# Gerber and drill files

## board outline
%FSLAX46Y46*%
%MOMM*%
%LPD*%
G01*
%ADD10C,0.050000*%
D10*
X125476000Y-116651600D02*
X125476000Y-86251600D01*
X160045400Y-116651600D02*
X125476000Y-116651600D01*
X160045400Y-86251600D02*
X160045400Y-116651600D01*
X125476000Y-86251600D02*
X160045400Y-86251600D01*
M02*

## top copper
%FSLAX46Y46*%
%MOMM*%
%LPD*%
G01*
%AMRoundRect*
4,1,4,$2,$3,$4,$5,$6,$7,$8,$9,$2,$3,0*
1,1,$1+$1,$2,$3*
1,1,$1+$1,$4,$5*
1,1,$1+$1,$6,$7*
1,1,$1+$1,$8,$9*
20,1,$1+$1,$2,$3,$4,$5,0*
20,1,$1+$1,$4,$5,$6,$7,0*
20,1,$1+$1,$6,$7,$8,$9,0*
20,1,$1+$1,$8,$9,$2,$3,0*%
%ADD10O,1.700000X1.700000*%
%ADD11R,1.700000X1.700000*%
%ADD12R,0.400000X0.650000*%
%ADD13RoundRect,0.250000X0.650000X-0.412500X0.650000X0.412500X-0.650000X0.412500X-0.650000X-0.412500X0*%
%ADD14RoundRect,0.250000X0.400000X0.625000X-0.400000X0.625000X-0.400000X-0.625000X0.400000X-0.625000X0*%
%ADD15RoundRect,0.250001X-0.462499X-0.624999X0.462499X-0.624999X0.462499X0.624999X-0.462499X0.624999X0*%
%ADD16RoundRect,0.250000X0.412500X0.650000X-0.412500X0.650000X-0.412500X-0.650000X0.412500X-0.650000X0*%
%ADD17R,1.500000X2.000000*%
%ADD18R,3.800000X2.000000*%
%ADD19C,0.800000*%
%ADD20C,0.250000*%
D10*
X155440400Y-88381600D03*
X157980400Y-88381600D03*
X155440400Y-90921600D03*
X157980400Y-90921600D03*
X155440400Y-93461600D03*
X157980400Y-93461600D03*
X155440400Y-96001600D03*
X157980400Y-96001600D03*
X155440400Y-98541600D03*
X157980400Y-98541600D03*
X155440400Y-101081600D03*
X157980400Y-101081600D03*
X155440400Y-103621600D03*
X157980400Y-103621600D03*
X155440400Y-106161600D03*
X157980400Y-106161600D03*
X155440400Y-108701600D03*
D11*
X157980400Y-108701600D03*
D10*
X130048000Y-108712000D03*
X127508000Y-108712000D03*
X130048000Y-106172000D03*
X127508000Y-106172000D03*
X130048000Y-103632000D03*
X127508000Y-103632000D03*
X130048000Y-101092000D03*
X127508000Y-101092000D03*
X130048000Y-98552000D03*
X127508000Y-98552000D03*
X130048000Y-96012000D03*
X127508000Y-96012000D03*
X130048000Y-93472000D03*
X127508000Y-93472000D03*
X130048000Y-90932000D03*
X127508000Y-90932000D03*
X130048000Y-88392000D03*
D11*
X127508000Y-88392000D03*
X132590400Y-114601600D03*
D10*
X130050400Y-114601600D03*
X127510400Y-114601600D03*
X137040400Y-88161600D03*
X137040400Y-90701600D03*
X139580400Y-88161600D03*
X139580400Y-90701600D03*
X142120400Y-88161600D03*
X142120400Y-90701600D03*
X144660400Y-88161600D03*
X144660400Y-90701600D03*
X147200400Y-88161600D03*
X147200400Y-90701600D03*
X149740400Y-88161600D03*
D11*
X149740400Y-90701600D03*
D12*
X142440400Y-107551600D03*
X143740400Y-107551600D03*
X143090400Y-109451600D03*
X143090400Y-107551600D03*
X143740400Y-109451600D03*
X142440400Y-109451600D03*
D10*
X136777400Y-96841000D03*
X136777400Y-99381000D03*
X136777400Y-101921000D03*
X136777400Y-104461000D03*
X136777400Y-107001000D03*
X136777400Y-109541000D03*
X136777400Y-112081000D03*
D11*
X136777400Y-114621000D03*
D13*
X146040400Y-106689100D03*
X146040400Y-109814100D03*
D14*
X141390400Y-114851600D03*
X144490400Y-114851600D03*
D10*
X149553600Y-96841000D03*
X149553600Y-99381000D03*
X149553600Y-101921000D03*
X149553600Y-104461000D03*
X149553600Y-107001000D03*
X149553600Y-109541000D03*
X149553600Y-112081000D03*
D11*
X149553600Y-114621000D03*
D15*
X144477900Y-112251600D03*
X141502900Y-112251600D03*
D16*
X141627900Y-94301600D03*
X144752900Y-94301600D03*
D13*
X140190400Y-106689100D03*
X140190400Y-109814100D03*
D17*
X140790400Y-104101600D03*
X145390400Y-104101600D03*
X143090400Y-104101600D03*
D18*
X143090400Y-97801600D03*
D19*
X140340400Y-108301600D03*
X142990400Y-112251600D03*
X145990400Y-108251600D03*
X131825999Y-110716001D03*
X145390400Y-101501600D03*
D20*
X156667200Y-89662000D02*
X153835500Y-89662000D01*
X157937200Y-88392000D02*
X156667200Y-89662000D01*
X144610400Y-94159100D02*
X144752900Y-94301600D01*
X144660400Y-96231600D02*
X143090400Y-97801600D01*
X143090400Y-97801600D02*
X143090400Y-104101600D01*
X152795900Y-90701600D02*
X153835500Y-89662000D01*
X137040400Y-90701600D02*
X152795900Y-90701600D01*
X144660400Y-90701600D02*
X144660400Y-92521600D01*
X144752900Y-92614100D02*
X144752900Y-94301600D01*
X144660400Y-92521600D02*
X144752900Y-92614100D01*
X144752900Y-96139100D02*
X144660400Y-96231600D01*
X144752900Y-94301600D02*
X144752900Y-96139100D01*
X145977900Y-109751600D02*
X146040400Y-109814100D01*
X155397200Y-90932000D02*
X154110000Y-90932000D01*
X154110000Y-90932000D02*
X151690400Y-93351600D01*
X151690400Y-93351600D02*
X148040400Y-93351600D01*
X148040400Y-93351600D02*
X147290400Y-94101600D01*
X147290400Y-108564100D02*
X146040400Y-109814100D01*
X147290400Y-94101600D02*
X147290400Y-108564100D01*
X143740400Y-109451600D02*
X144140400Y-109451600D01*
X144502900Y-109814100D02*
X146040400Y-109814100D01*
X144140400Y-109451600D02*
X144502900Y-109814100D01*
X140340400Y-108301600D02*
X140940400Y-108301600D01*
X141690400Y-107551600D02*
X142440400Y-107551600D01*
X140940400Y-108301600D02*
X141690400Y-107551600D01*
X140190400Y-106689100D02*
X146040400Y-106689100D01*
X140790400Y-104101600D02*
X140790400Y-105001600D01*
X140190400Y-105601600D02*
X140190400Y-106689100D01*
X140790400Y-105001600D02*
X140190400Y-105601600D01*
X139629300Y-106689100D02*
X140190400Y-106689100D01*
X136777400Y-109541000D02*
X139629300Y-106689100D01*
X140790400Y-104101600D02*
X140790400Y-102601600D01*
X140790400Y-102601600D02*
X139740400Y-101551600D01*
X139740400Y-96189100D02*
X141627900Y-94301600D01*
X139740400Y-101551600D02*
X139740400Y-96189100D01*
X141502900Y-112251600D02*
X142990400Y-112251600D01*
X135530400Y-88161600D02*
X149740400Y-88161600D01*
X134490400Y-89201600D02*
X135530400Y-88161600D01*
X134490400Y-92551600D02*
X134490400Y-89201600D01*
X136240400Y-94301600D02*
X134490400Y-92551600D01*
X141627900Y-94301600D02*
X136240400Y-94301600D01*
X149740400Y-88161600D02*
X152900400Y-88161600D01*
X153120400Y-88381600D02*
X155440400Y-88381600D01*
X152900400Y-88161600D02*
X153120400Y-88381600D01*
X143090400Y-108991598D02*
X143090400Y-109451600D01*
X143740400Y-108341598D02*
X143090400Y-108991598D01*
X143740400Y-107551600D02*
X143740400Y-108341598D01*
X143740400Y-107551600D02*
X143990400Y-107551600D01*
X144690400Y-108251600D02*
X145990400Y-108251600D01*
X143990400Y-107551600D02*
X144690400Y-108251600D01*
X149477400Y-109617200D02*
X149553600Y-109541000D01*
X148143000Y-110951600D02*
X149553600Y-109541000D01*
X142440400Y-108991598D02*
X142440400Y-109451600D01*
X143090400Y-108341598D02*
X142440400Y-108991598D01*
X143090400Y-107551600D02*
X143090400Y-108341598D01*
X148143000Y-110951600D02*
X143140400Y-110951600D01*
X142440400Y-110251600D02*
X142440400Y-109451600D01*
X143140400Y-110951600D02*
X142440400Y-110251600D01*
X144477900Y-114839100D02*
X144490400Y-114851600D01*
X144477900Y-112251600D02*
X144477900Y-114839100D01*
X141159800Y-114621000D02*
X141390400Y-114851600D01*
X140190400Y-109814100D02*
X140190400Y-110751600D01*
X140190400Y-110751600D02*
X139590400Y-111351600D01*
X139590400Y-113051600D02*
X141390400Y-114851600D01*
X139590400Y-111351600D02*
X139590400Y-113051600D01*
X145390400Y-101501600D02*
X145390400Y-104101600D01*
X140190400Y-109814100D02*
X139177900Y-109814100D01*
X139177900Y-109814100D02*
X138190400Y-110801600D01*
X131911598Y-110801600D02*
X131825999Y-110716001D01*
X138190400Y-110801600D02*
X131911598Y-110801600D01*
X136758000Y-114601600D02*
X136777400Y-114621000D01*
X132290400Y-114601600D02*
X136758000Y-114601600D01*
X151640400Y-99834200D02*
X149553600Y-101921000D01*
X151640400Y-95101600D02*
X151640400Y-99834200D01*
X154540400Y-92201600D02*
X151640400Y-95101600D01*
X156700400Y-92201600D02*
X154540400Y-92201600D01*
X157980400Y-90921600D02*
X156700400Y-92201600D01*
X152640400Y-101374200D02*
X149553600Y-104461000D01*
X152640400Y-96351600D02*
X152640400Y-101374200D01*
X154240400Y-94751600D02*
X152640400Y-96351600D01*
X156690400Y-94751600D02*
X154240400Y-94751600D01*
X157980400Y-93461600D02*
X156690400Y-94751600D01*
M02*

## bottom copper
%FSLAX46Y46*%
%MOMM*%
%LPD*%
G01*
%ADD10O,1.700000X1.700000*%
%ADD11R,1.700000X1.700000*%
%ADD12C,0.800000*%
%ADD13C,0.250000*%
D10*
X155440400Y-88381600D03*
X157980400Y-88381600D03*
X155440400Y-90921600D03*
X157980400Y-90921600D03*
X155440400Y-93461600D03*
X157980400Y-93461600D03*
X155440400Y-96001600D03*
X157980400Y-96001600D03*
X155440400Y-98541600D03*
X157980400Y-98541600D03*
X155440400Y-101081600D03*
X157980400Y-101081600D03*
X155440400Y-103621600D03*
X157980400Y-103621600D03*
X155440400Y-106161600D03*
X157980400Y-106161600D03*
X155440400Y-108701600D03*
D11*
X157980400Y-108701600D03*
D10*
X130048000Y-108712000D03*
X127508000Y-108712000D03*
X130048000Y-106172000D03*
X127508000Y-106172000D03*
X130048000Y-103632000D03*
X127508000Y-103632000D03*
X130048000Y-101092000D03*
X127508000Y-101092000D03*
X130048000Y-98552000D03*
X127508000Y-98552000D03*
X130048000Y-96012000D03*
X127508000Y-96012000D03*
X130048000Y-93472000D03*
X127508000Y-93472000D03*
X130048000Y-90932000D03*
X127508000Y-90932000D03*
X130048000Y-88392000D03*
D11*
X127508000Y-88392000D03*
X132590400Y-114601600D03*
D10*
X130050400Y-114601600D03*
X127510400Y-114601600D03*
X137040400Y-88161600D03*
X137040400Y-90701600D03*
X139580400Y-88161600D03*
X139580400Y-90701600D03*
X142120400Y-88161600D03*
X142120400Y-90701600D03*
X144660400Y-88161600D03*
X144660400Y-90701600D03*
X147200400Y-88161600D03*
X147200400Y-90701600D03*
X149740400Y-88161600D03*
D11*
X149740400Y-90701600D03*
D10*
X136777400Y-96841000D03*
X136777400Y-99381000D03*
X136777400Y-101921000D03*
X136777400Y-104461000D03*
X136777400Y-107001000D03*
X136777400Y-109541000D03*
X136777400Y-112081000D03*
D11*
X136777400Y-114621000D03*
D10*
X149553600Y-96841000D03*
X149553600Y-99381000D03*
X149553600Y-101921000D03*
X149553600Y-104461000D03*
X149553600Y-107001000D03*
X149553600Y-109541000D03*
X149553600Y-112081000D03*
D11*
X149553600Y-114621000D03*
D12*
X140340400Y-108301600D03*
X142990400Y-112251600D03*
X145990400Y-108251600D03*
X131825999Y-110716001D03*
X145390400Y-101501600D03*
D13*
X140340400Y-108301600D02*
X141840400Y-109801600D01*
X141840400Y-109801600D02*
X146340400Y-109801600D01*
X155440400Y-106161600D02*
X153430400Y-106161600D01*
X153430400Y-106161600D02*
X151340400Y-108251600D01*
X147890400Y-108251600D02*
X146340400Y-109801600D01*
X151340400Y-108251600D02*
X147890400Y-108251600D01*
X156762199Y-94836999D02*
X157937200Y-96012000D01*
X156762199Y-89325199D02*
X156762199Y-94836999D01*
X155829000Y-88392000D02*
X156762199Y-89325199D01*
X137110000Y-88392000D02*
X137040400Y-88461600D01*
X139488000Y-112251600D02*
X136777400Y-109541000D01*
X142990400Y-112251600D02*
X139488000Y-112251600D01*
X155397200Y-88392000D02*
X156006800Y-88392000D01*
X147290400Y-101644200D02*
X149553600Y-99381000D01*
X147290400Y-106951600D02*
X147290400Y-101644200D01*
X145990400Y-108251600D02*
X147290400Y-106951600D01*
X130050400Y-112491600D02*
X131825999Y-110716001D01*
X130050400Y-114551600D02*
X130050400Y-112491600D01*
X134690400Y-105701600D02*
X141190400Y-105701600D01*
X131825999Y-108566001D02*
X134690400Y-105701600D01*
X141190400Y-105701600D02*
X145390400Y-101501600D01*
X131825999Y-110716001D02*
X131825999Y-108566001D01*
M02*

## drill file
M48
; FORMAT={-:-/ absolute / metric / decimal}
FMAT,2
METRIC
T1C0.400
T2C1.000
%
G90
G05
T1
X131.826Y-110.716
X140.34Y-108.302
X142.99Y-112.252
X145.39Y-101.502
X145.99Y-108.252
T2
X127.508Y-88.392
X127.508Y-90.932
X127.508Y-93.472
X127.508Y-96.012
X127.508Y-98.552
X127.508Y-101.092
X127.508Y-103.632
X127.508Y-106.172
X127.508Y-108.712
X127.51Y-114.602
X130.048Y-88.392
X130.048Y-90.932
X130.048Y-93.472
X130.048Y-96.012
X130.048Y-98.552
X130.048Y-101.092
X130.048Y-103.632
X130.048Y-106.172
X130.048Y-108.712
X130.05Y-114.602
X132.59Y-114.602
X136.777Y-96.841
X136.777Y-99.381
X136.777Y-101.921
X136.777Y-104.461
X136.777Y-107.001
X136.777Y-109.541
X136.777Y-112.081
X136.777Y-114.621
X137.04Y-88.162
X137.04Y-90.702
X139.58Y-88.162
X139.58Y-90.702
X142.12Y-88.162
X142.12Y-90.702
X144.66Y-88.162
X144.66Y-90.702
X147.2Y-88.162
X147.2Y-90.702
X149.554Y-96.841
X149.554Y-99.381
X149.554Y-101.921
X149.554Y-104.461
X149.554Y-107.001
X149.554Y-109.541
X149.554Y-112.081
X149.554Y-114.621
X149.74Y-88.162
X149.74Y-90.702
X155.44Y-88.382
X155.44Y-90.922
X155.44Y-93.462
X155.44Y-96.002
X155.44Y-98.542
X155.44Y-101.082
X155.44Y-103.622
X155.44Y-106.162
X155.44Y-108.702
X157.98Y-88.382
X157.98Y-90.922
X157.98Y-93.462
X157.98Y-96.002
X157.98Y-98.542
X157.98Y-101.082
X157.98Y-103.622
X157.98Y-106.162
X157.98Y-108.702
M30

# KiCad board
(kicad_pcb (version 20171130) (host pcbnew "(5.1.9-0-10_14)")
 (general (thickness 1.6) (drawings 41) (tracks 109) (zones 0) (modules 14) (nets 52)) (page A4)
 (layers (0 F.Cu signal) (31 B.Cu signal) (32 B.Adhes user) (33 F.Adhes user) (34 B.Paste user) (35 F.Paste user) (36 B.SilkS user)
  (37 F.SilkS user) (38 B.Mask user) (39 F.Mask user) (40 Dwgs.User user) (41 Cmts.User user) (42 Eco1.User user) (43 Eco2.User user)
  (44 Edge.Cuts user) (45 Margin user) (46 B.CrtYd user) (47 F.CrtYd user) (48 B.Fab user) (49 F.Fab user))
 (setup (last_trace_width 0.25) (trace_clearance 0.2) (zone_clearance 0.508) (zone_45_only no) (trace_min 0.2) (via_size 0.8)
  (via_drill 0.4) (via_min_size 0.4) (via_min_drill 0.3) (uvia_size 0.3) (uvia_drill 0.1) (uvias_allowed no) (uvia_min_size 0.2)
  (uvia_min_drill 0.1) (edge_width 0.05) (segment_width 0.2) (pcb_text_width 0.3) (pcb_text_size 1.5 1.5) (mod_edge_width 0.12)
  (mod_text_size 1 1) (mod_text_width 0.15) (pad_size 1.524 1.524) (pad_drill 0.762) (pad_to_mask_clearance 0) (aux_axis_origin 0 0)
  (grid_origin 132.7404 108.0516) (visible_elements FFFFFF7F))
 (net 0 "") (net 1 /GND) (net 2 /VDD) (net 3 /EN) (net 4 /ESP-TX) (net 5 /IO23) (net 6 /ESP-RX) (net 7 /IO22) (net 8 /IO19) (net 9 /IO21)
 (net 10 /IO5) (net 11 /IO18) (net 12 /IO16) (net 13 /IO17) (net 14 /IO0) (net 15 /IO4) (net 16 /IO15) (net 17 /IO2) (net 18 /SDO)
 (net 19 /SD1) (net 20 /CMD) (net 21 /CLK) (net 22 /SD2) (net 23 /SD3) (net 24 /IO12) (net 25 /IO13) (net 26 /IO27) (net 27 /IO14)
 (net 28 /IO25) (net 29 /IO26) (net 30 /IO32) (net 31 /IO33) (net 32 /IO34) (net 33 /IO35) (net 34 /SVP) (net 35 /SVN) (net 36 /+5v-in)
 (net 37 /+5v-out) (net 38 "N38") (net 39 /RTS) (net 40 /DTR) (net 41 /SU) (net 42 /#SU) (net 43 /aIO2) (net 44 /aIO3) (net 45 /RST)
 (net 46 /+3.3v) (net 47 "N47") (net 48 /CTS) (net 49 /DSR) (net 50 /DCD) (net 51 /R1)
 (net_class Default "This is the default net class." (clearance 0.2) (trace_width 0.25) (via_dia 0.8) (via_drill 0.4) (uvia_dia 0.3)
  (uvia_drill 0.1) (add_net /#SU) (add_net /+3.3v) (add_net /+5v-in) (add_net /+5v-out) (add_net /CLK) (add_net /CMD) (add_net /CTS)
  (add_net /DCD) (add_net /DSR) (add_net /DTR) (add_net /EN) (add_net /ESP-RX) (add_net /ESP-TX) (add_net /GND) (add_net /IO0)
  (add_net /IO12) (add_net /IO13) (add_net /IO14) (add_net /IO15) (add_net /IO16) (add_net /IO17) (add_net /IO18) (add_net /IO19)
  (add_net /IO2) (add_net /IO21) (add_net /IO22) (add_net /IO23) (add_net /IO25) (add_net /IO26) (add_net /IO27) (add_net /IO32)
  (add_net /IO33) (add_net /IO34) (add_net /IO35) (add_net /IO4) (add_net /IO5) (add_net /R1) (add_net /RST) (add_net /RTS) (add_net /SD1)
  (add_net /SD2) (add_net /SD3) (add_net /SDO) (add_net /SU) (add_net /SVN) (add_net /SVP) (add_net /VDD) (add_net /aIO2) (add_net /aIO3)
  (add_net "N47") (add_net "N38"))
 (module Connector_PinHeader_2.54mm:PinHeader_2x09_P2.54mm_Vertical (layer F.Cu) (at 157.9804 108.7016 180)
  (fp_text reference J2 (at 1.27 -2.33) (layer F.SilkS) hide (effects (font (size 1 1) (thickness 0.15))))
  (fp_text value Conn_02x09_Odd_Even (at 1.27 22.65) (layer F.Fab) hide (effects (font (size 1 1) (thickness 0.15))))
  (pad 18 thru_hole oval (at 2.54 20.32 180) (size 1.7 1.7) (drill 1) (layers *.Cu *.Mask) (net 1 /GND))
  (pad 17 thru_hole oval (at 0 20.32 180) (size 1.7 1.7) (drill 1) (layers *.Cu *.Mask) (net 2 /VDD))
  (pad 16 thru_hole oval (at 2.54 17.78 180) (size 1.7 1.7) (drill 1) (layers *.Cu *.Mask) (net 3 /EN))
  (pad 15 thru_hole oval (at 0 17.78 180) (size 1.7 1.7) (drill 1) (layers *.Cu *.Mask) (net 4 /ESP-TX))
  (pad 14 thru_hole oval (at 2.54 15.24 180) (size 1.7 1.7) (drill 1) (layers *.Cu *.Mask) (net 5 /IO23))
  (pad 13 thru_hole oval (at 0 15.24 180) (size 1.7 1.7) (drill 1) (layers *.Cu *.Mask) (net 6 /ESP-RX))
  (pad 12 thru_hole oval (at 2.54 12.7 180) (size 1.7 1.7) (drill 1) (layers *.Cu *.Mask) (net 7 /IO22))
  (pad 11 thru_hole oval (at 0 12.7 180) (size 1.7 1.7) (drill 1) (layers *.Cu *.Mask) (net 1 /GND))
  (pad 10 thru_hole oval (at 2.54 10.16 180) (size 1.7 1.7) (drill 1) (layers *.Cu *.Mask) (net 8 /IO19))
  (pad 9 thru_hole oval (at 0 10.16 180) (size 1.7 1.7) (drill 1) (layers *.Cu *.Mask) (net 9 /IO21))
  (pad 8 thru_hole oval (at 2.54 7.62 180) (size 1.7 1.7) (drill 1) (layers *.Cu *.Mask) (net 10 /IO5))
  (pad 7 thru_hole oval (at 0 7.62 180) (size 1.7 1.7) (drill 1) (layers *.Cu *.Mask) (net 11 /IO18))
  (pad 6 thru_hole oval (at 2.54 5.08 180) (size 1.7 1.7) (drill 1) (layers *.Cu *.Mask) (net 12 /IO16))
  (pad 5 thru_hole oval (at 0 5.08 180) (size 1.7 1.7) (drill 1) (layers *.Cu *.Mask) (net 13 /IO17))
  (pad 4 thru_hole oval (at 2.54 2.54 180) (size 1.7 1.7) (drill 1) (layers *.Cu *.Mask) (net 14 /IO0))
  (pad 3 thru_hole oval (at 0 2.54 180) (size 1.7 1.7) (drill 1) (layers *.Cu *.Mask) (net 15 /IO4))
  (pad 2 thru_hole oval (at 2.54 0 180) (size 1.7 1.7) (drill 1) (layers *.Cu *.Mask) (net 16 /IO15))
  (pad 1 thru_hole rect (at 0 0 180) (size 1.7 1.7) (drill 1) (layers *.Cu *.Mask) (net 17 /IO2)))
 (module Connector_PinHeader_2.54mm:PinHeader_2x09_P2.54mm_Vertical (layer F.Cu) (at 127.508 88.392)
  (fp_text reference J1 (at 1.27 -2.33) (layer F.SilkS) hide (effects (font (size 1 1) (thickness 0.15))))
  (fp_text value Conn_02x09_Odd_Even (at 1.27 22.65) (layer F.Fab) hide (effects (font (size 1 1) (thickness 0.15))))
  (pad 18 thru_hole oval (at 2.54 20.32) (size 1.7 1.7) (drill 1) (layers *.Cu *.Mask) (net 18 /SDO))
  (pad 17 thru_hole oval (at 0 20.32) (size 1.7 1.7) (drill 1) (layers *.Cu *.Mask) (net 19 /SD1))
  (pad 16 thru_hole oval (at 2.54 17.78) (size 1.7 1.7) (drill 1) (layers *.Cu *.Mask) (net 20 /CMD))
  (pad 15 thru_hole oval (at 0 17.78) (size 1.7 1.7) (drill 1) (layers *.Cu *.Mask) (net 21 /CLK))
  (pad 14 thru_hole oval (at 2.54 15.24) (size 1.7 1.7) (drill 1) (layers *.Cu *.Mask) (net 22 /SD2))
  (pad 13 thru_hole oval (at 0 15.24) (size 1.7 1.7) (drill 1) (layers *.Cu *.Mask) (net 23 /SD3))
  (pad 12 thru_hole oval (at 2.54 12.7) (size 1.7 1.7) (drill 1) (layers *.Cu *.Mask) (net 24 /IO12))
  (pad 11 thru_hole oval (at 0 12.7) (size 1.7 1.7) (drill 1) (layers *.Cu *.Mask) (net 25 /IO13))
  (pad 10 thru_hole oval (at 2.54 10.16) (size 1.7 1.7) (drill 1) (layers *.Cu *.Mask) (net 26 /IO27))
  (pad 9 thru_hole oval (at 0 10.16) (size 1.7 1.7) (drill 1) (layers *.Cu *.Mask) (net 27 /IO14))
  (pad 8 thru_hole oval (at 2.54 7.62) (size 1.7 1.7) (drill 1) (layers *.Cu *.Mask) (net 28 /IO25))
  (pad 7 thru_hole oval (at 0 7.62) (size 1.7 1.7) (drill 1) (layers *.Cu *.Mask) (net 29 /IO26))
  (pad 6 thru_hole oval (at 2.54 5.08) (size 1.7 1.7) (drill 1) (layers *.Cu *.Mask) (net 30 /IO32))
  (pad 5 thru_hole oval (at 0 5.08) (size 1.7 1.7) (drill 1) (layers *.Cu *.Mask) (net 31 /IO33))
  (pad 4 thru_hole oval (at 2.54 2.54) (size 1.7 1.7) (drill 1) (layers *.Cu *.Mask) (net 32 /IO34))
  (pad 3 thru_hole oval (at 0 2.54) (size 1.7 1.7) (drill 1) (layers *.Cu *.Mask) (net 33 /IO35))
  (pad 2 thru_hole oval (at 2.54 0) (size 1.7 1.7) (drill 1) (layers *.Cu *.Mask) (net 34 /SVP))
  (pad 1 thru_hole rect (at 0 0) (size 1.7 1.7) (drill 1) (layers *.Cu *.Mask) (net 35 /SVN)))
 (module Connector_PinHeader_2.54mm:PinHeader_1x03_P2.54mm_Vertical (layer B.Cu) (at 132.5904 114.6016 90)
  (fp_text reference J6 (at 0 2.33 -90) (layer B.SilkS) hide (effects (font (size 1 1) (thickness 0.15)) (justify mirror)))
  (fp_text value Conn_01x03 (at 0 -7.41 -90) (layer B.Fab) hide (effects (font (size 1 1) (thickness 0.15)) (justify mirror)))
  (pad 1 thru_hole rect (at 0 0 90) (size 1.7 1.7) (drill 1) (layers *.Cu *.Mask) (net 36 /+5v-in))
  (pad 2 thru_hole oval (at 0 -2.54 90) (size 1.7 1.7) (drill 1) (layers *.Cu *.Mask) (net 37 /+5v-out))
  (pad 3 thru_hole oval (at 0 -5.08 90) (size 1.7 1.7) (drill 1) (layers *.Cu *.Mask) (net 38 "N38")))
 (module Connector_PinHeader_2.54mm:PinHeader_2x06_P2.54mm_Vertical (layer B.Cu) (at 149.7404 90.7016 90)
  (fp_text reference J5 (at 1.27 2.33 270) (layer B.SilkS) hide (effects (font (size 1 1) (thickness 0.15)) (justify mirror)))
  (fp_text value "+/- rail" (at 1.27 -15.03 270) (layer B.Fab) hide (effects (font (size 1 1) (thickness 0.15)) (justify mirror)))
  (pad 12 thru_hole oval (at 2.54 -12.7 90) (size 1.7 1.7) (drill 1) (layers *.Cu *.Mask) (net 1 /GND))
  (pad 11 thru_hole oval (at 0 -12.7 90) (size 1.7 1.7) (drill 1) (layers *.Cu *.Mask) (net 2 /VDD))
  (pad 10 thru_hole oval (at 2.54 -10.16 90) (size 1.7 1.7) (drill 1) (layers *.Cu *.Mask) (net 1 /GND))
  (pad 9 thru_hole oval (at 0 -10.16 90) (size 1.7 1.7) (drill 1) (layers *.Cu *.Mask) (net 2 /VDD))
  (pad 8 thru_hole oval (at 2.54 -7.62 90) (size 1.7 1.7) (drill 1) (layers *.Cu *.Mask) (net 1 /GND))
  (pad 7 thru_hole oval (at 0 -7.62 90) (size 1.7 1.7) (drill 1) (layers *.Cu *.Mask) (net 2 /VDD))
  (pad 6 thru_hole oval (at 2.54 -5.08 90) (size 1.7 1.7) (drill 1) (layers *.Cu *.Mask) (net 1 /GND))
  (pad 5 thru_hole oval (at 0 -5.08 90) (size 1.7 1.7) (drill 1) (layers *.Cu *.Mask) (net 2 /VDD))
  (pad 4 thru_hole oval (at 2.54 -2.54 90) (size 1.7 1.7) (drill 1) (layers *.Cu *.Mask) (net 1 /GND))
  (pad 3 thru_hole oval (at 0 -2.54 90) (size 1.7 1.7) (drill 1) (layers *.Cu *.Mask) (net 2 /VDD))
  (pad 2 thru_hole oval (at 2.54 0 90) (size 1.7 1.7) (drill 1) (layers *.Cu *.Mask) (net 1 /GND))
  (pad 1 thru_hole rect (at 0 0 90) (size 1.7 1.7) (drill 1) (layers *.Cu *.Mask) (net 2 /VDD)))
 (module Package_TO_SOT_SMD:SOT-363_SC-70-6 (layer F.Cu) (at 143.0904 108.5016 90)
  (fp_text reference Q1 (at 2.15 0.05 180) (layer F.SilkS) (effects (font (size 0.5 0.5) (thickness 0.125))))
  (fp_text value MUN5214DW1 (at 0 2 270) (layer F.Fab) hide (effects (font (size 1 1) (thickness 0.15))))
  (pad 6 smd rect (at 0.95 -0.65 90) (size 0.65 0.4) (layers F.Cu F.Paste F.Mask) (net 14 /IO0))
  (pad 4 smd rect (at 0.95 0.65 90) (size 0.65 0.4) (layers F.Cu F.Paste F.Mask) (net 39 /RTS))
  (pad 2 smd rect (at -0.95 0 90) (size 0.65 0.4) (layers F.Cu F.Paste F.Mask) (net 39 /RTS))
  (pad 5 smd rect (at 0.95 0 90) (size 0.65 0.4) (layers F.Cu F.Paste F.Mask) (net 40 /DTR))
  (pad 3 smd rect (at -0.95 0.65 90) (size 0.65 0.4) (layers F.Cu F.Paste F.Mask) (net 3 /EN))
  (pad 1 smd rect (at -0.95 -0.65 90) (size 0.65 0.4) (layers F.Cu F.Paste F.Mask) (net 40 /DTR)))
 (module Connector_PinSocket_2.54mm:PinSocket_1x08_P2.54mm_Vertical (layer B.Cu) (at 136.7774 114.621)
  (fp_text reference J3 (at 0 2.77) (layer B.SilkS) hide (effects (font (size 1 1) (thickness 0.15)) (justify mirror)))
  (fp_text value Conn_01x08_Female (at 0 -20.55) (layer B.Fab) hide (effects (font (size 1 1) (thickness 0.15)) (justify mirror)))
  (pad 8 thru_hole oval (at 0 -17.78) (size 1.7 1.7) (drill 1) (layers *.Cu *.Mask) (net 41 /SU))
  (pad 7 thru_hole oval (at 0 -15.24) (size 1.7 1.7) (drill 1) (layers *.Cu *.Mask) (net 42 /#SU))
  (pad 6 thru_hole oval (at 0 -12.7) (size 1.7 1.7) (drill 1) (layers *.Cu *.Mask) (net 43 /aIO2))
  (pad 5 thru_hole oval (at 0 -10.16) (size 1.7 1.7) (drill 1) (layers *.Cu *.Mask) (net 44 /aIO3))
  (pad 4 thru_hole oval (at 0 -7.62) (size 1.7 1.7) (drill 1) (layers *.Cu *.Mask) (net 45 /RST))
  (pad 3 thru_hole oval (at 0 -5.08) (size 1.7 1.7) (drill 1) (layers *.Cu *.Mask) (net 1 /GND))
  (pad 2 thru_hole oval (at 0 -2.54) (size 1.7 1.7) (drill 1) (layers *.Cu *.Mask) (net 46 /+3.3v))
  (pad 1 thru_hole rect (at 0 0) (size 1.7 1.7) (drill 1) (layers *.Cu *.Mask) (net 36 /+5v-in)))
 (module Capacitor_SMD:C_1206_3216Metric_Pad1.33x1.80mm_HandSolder (layer F.Cu) (at 146.0404 108.2516 90)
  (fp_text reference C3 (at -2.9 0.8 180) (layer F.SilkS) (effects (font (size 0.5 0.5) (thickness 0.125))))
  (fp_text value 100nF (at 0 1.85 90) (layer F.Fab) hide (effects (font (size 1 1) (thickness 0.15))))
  (pad 2 smd roundrect (at 1.5625 0 90) (size 1.325 1.8) (layers F.Cu F.Paste F.Mask) (roundrect_rratio 0.188679) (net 1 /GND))
  (pad 1 smd roundrect (at -1.5625 0 90) (size 1.325 1.8) (layers F.Cu F.Paste F.Mask) (roundrect_rratio 0.188679) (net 3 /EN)))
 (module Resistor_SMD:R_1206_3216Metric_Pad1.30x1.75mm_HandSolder (layer F.Cu) (at 142.9404 114.8516 180)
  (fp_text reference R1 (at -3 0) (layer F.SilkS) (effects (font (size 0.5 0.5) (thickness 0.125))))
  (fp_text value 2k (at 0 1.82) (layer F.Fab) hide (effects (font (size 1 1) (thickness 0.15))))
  (pad 2 smd roundrect (at 1.55 0 180) (size 1.3 1.75) (layers F.Cu F.Paste F.Mask) (roundrect_rratio 0.192308) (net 37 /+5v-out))
  (pad 1 smd roundrect (at -1.55 0 180) (size 1.3 1.75) (layers F.Cu F.Paste F.Mask) (roundrect_rratio 0.192308) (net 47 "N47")))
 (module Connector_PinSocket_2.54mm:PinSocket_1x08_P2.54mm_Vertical (layer B.Cu) (at 149.5536 114.621)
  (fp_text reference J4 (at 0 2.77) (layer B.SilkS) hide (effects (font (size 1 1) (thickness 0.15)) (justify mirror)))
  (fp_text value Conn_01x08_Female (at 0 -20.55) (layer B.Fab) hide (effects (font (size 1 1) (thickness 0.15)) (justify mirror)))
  (pad 8 thru_hole oval (at 0 -17.78) (size 1.7 1.7) (drill 1) (layers *.Cu *.Mask) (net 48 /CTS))
  (pad 7 thru_hole oval (at 0 -15.24) (size 1.7 1.7) (drill 1) (layers *.Cu *.Mask) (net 39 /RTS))
  (pad 6 thru_hole oval (at 0 -12.7) (size 1.7 1.7) (drill 1) (layers *.Cu *.Mask) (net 4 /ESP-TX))
  (pad 5 thru_hole oval (at 0 -10.16) (size 1.7 1.7) (drill 1) (layers *.Cu *.Mask) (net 6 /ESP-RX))
  (pad 4 thru_hole oval (at 0 -7.62) (size 1.7 1.7) (drill 1) (layers *.Cu *.Mask) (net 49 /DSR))
  (pad 3 thru_hole oval (at 0 -5.08) (size 1.7 1.7) (drill 1) (layers *.Cu *.Mask) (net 40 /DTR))
  (pad 2 thru_hole oval (at 0 -2.54) (size 1.7 1.7) (drill 1) (layers *.Cu *.Mask) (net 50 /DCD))
  (pad 1 thru_hole rect (at 0 0) (size 1.7 1.7) (drill 1) (layers *.Cu *.Mask) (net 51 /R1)))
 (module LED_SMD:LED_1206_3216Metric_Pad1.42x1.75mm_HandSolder (layer F.Cu) (at 142.9904 112.2516)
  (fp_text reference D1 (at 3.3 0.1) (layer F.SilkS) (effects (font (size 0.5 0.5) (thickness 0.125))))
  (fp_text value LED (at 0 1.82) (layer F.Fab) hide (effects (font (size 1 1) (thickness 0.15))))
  (pad 2 smd roundrect (at 1.4875 0) (size 1.425 1.75) (layers F.Cu F.Paste F.Mask) (roundrect_rratio 0.175439) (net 47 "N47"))
  (pad 1 smd roundrect (at -1.4875 0) (size 1.425 1.75) (layers F.Cu F.Paste F.Mask) (roundrect_rratio 0.175439) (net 1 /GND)))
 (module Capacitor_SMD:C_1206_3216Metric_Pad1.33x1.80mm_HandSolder (layer F.Cu) (at 143.1904 94.3016 180)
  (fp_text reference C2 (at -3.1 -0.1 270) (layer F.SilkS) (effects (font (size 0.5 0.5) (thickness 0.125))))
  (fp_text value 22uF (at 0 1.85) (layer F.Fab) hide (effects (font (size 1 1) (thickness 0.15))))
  (pad 2 smd roundrect (at 1.5625 0 180) (size 1.325 1.8) (layers F.Cu F.Paste F.Mask) (roundrect_rratio 0.188679) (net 1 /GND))
  (pad 1 smd roundrect (at -1.5625 0 180) (size 1.325 1.8) (layers F.Cu F.Paste F.Mask) (roundrect_rratio 0.188679) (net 2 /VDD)))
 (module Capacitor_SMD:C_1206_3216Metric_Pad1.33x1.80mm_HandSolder (layer F.Cu) (at 140.1904 108.2516 90)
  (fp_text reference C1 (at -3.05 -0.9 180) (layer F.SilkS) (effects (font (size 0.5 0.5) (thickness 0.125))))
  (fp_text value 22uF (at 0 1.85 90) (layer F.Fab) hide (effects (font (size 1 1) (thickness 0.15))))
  (pad 2 smd roundrect (at 1.5625 0 90) (size 1.325 1.8) (layers F.Cu F.Paste F.Mask) (roundrect_rratio 0.188679) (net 1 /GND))
  (pad 1 smd roundrect (at -1.5625 0 90) (size 1.325 1.8) (layers F.Cu F.Paste F.Mask) (roundrect_rratio 0.188679) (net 37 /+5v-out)))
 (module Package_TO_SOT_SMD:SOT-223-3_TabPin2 (layer F.Cu) (at 143.0904 100.9516 90)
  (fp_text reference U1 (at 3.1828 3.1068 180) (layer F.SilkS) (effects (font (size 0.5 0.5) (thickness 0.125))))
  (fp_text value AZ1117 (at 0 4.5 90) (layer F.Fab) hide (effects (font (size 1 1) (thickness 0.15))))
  (pad 1 smd rect (at -3.15 -2.3 90) (size 2 1.5) (layers F.Cu F.Paste F.Mask) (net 1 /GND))
  (pad 3 smd rect (at -3.15 2.3 90) (size 2 1.5) (layers F.Cu F.Paste F.Mask) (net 37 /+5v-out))
  (pad 2 smd rect (at -3.15 0 90) (size 2 1.5) (layers F.Cu F.Paste F.Mask) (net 2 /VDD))
  (pad 2 smd rect (at 3.15 0 90) (size 2 3.8) (layers F.Cu F.Paste F.Mask) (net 2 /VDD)))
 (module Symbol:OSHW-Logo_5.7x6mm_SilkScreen (layer B.Cu) (at 143.5404 95.6016 180)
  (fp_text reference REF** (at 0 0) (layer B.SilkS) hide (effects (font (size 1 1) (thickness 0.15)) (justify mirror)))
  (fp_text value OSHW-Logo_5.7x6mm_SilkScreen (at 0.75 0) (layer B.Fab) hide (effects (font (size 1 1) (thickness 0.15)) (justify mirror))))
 (gr_line (start 125.476 116.6516) (end 125.476 86.2516) (layer Edge.Cuts) (width 0.05))
 (gr_line (start 160.0454 116.6516) (end 125.476 116.6516) (layer Edge.Cuts) (width 0.05))
 (gr_line (start 160.0454 86.2516) (end 160.0454 116.6516) (layer Edge.Cuts) (width 0.05))
 (gr_line (start 125.476 86.2516) (end 160.0454 86.2516) (layer Edge.Cuts) (width 0.05))
 (segment (start 156.6672 89.662) (end 153.8355 89.662) (width 0.25) (layer F.Cu) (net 2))
 (segment (start 157.9372 88.392) (end 156.6672 89.662) (width 0.25) (layer F.Cu) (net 2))
 (segment (start 144.6104 94.1591) (end 144.7529 94.3016) (width 0.25) (layer F.Cu) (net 2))
 (segment (start 144.6604 96.2316) (end 143.0904 97.8016) (width 0.25) (layer F.Cu) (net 2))
 (segment (start 143.0904 97.8016) (end 143.0904 104.1016) (width 0.25) (layer F.Cu) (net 2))
 (segment (start 152.7959 90.7016) (end 153.8355 89.662) (width 0.25) (layer F.Cu) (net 2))
 (segment (start 137.0404 90.7016) (end 152.7959 90.7016) (width 0.25) (layer F.Cu) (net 2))
 (segment (start 144.6604 90.7016) (end 144.6604 92.5216) (width 0.25) (layer F.Cu) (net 2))
 (segment (start 144.7529 92.6141) (end 144.7529 94.3016) (width 0.25) (layer F.Cu) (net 2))
 (segment (start 144.6604 92.5216) (end 144.7529 92.6141) (width 0.25) (layer F.Cu) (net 2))
 (segment (start 144.7529 96.1391) (end 144.6604 96.2316) (width 0.25) (layer F.Cu) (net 2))
 (segment (start 144.7529 94.3016) (end 144.7529 96.1391) (width 0.25) (layer F.Cu) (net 2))
 (segment (start 145.9779 109.7516) (end 146.0404 109.8141) (width 0.25) (layer F.Cu) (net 3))
 (segment (start 155.3972 90.932) (end 154.11 90.932) (width 0.25) (layer F.Cu) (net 3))
 (segment (start 154.11 90.932) (end 151.6904 93.3516) (width 0.25) (layer F.Cu) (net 3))
 (segment (start 151.6904 93.3516) (end 148.0404 93.3516) (width 0.25) (layer F.Cu) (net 3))
 (segment (start 148.0404 93.3516) (end 147.2904 94.1016) (width 0.25) (layer F.Cu) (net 3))
 (segment (start 147.2904 108.5641) (end 146.0404 109.8141) (width 0.25) (layer F.Cu) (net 3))
 (segment (start 147.2904 94.1016) (end 147.2904 108.5641) (width 0.25) (layer F.Cu) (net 3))
 (segment (start 143.7404 109.4516) (end 144.1404 109.4516) (width 0.25) (layer F.Cu) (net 3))
 (segment (start 144.5029 109.8141) (end 146.0404 109.8141) (width 0.25) (layer F.Cu) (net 3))
 (segment (start 144.1404 109.4516) (end 144.5029 109.8141) (width 0.25) (layer F.Cu) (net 3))
 (via (at 140.3404 108.3016) (size 0.8) (drill 0.4) (layers F.Cu B.Cu) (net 14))
 (segment (start 140.3404 108.3016) (end 141.8404 109.8016) (width 0.25) (layer B.Cu) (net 14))
 (segment (start 141.8404 109.8016) (end 146.3404 109.8016) (width 0.25) (layer B.Cu) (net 14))
 (segment (start 140.3404 108.3016) (end 140.9404 108.3016) (width 0.25) (layer F.Cu) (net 14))
 (segment (start 141.6904 107.5516) (end 142.4404 107.5516) (width 0.25) (layer F.Cu) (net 14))
 (segment (start 140.9404 108.3016) (end 141.6904 107.5516) (width 0.25) (layer F.Cu) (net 14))
 (segment (start 155.4404 106.1616) (end 153.4304 106.1616) (width 0.25) (layer B.Cu) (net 14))
 (segment (start 153.4304 106.1616) (end 151.3404 108.2516) (width 0.25) (layer B.Cu) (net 14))
 (segment (start 147.8904 108.2516) (end 146.3404 109.8016) (width 0.25) (layer B.Cu) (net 14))
 (segment (start 151.3404 108.2516) (end 147.8904 108.2516) (width 0.25) (layer B.Cu) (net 14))
 (segment (start 156.762199 94.836999) (end 157.9372 96.012) (width 0.25) (layer B.Cu) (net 1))
 (segment (start 156.762199 89.325199) (end 156.762199 94.836999) (width 0.25) (layer B.Cu) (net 1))
 (segment (start 155.829 88.392) (end 156.762199 89.325199) (width 0.25) (layer B.Cu) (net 1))
 (segment (start 137.11 88.392) (end 137.0404 88.4616) (width 0.25) (layer B.Cu) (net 1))
 (segment (start 140.1904 106.6891) (end 146.0404 106.6891) (width 0.25) (layer F.Cu) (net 1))
 (segment (start 140.7904 104.1016) (end 140.7904 105.0016) (width 0.25) (layer F.Cu) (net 1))
 (segment (start 140.1904 105.6016) (end 140.1904 106.6891) (width 0.25) (layer F.Cu) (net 1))
 (segment (start 140.7904 105.0016) (end 140.1904 105.6016) (width 0.25) (layer F.Cu) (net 1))
 (segment (start 139.6293 106.6891) (end 140.1904 106.6891) (width 0.25) (layer F.Cu) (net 1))
 (segment (start 136.7774 109.541) (end 139.6293 106.6891) (width 0.25) (layer F.Cu) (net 1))
 (segment (start 140.7904 104.1016) (end 140.7904 102.6016) (width 0.25) (layer F.Cu) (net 1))
 (segment (start 140.7904 102.6016) (end 139.7404 101.5516) (width 0.25) (layer F.Cu) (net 1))
 (segment (start 139.7404 96.1891) (end 141.6279 94.3016) (width 0.25) (layer F.Cu) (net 1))
 (segment (start 139.7404 101.5516) (end 139.7404 96.1891) (width 0.25) (layer F.Cu) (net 1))
 (via (at 142.9904 112.2516) (size 0.8) (drill 0.4) (layers F.Cu B.Cu) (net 1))
 (segment (start 141.5029 112.2516) (end 142.9904 112.2516) (width 0.25) (layer F.Cu) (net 1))
 (segment (start 139.488 112.2516) (end 136.7774 109.541) (width 0.25) (layer B.Cu) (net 1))
 (segment (start 142.9904 112.2516) (end 139.488 112.2516) (width 0.25) (layer B.Cu) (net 1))
 (segment (start 155.3972 88.392) (end 156.0068 88.392) (width 0.25) (layer B.Cu) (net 1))
 (segment (start 135.5304 88.1616) (end 149.7404 88.1616) (width 0.25) (layer F.Cu) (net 1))
 (segment (start 134.4904 89.2016) (end 135.5304 88.1616) (width 0.25) (layer F.Cu) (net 1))
 (segment (start 134.4904 92.5516) (end 134.4904 89.2016) (width 0.25) (layer F.Cu) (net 1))
 (segment (start 136.2404 94.3016) (end 134.4904 92.5516) (width 0.25) (layer F.Cu) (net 1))
 (segment (start 141.6279 94.3016) (end 136.2404 94.3016) (width 0.25) (layer F.Cu) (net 1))
 (segment (start 149.7404 88.1616) (end 152.9004 88.1616) (width 0.25) (layer F.Cu) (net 1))
 (segment (start 153.1204 88.3816) (end 155.4404 88.3816) (width 0.25) (layer F.Cu) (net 1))
 (segment (start 152.9004 88.1616) (end 153.1204 88.3816) (width 0.25) (layer F.Cu) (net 1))
 (segment (start 143.0904 108.991598) (end 143.0904 109.4516) (width 0.25) (layer F.Cu) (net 39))
 (segment (start 143.7404 108.341598) (end 143.0904 108.991598) (width 0.25) (layer F.Cu) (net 39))
 (segment (start 143.7404 107.5516) (end 143.7404 108.341598) (width 0.25) (layer F.Cu) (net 39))
 (segment (start 143.7404 107.5516) (end 143.9904 107.5516) (width 0.25) (layer F.Cu) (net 39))
 (via (at 145.9904 108.2516) (size 0.8) (drill 0.4) (layers F.Cu B.Cu) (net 39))
 (segment (start 144.6904 108.2516) (end 145.9904 108.2516) (width 0.25) (layer F.Cu) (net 39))
 (segment (start 143.9904 107.5516) (end 144.6904 108.2516) (width 0.25) (layer F.Cu) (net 39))
 (segment (start 147.2904 101.6442) (end 149.5536 99.381) (width 0.25) (layer B.Cu) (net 39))
 (segment (start 147.2904 106.9516) (end 147.2904 101.6442) (width 0.25) (layer B.Cu) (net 39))
 (segment (start 145.9904 108.2516) (end 147.2904 106.9516) (width 0.25) (layer B.Cu) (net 39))
 (segment (start 149.4774 109.6172) (end 149.5536 109.541) (width 0.25) (layer F.Cu) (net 40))
 (segment (start 148.143 110.9516) (end 149.5536 109.541) (width 0.25) (layer F.Cu) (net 40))
 (segment (start 142.4404 108.991598) (end 142.4404 109.4516) (width 0.25) (layer F.Cu) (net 40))
 (segment (start 143.0904 108.341598) (end 142.4404 108.991598) (width 0.25) (layer F.Cu) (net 40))
 (segment (start 143.0904 107.5516) (end 143.0904 108.341598) (width 0.25) (layer F.Cu) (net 40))
 (segment (start 148.143 110.9516) (end 143.1404 110.9516) (width 0.25) (layer F.Cu) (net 40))
 (segment (start 142.4404 110.2516) (end 142.4404 109.4516) (width 0.25) (layer F.Cu) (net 40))
 (segment (start 143.1404 110.9516) (end 142.4404 110.2516) (width 0.25) (layer F.Cu) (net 40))
 (segment (start 144.4779 114.8391) (end 144.4904 114.8516) (width 0.25) (layer F.Cu) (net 47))
 (segment (start 144.4779 112.2516) (end 144.4779 114.8391) (width 0.25) (layer F.Cu) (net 47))
 (segment (start 141.1598 114.621) (end 141.3904 114.8516) (width 0.25) (layer F.Cu) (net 37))
 (segment (start 140.1904 109.8141) (end 140.1904 110.7516) (width 0.25) (layer F.Cu) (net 37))
 (segment (start 140.1904 110.7516) (end 139.5904 111.3516) (width 0.25) (layer F.Cu) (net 37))
 (segment (start 139.5904 113.0516) (end 141.3904 114.8516) (width 0.25) (layer F.Cu) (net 37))
 (segment (start 139.5904 111.3516) (end 139.5904 113.0516) (width 0.25) (layer F.Cu) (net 37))
 (via (at 131.825999 110.716001) (size 0.8) (drill 0.4) (layers F.Cu B.Cu) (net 37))
 (via (at 145.3904 101.5016) (size 0.8) (drill 0.4) (layers F.Cu B.Cu) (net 37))
 (segment (start 145.3904 101.5016) (end 145.3904 104.1016) (width 0.25) (layer F.Cu) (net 37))
 (segment (start 130.0504 112.4916) (end 131.825999 110.716001) (width 0.25) (layer B.Cu) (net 37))
 (segment (start 130.0504 114.5516) (end 130.0504 112.4916) (width 0.25) (layer B.Cu) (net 37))
 (segment (start 134.6904 105.7016) (end 141.1904 105.7016) (width 0.25) (layer B.Cu) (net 37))
 (segment (start 131.825999 108.566001) (end 134.6904 105.7016) (width 0.25) (layer B.Cu) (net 37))
 (segment (start 141.1904 105.7016) (end 145.3904 101.5016) (width 0.25) (layer B.Cu) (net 37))
 (segment (start 131.825999 110.716001) (end 131.825999 108.566001) (width 0.25) (layer B.Cu) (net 37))
 (segment (start 140.1904 109.8141) (end 139.1779 109.8141) (width 0.25) (layer F.Cu) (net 37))
 (segment (start 139.1779 109.8141) (end 138.1904 110.8016) (width 0.25) (layer F.Cu) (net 37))
 (segment (start 131.911598 110.8016) (end 131.825999 110.716001) (width 0.25) (layer F.Cu) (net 37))
 (segment (start 138.1904 110.8016) (end 131.911598 110.8016) (width 0.25) (layer F.Cu) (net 37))
 (segment (start 136.758 114.6016) (end 136.7774 114.621) (width 0.25) (layer F.Cu) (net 36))
 (segment (start 132.2904 114.6016) (end 136.758 114.6016) (width 0.25) (layer F.Cu) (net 36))
 (segment (start 151.6404 99.8342) (end 149.5536 101.921) (width 0.25) (layer F.Cu) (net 4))
 (segment (start 151.6404 95.1016) (end 151.6404 99.8342) (width 0.25) (layer F.Cu) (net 4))
 (segment (start 154.5404 92.2016) (end 151.6404 95.1016) (width 0.25) (layer F.Cu) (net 4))
 (segment (start 156.7004 92.2016) (end 154.5404 92.2016) (width 0.25) (layer F.Cu) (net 4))
 (segment (start 157.9804 90.9216) (end 156.7004 92.2016) (width 0.25) (layer F.Cu) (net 4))
 (segment (start 152.6404 101.3742) (end 149.5536 104.461) (width 0.25) (layer F.Cu) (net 6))
 (segment (start 152.6404 96.3516) (end 152.6404 101.3742) (width 0.25) (layer F.Cu) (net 6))
 (segment (start 154.2404 94.7516) (end 152.6404 96.3516) (width 0.25) (layer F.Cu) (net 6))
 (segment (start 156.6904 94.7516) (end 154.2404 94.7516) (width 0.25) (layer F.Cu) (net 6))
 (segment (start 157.9804 93.4616) (end 156.6904 94.7516) (width 0.25) (layer F.Cu) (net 6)))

